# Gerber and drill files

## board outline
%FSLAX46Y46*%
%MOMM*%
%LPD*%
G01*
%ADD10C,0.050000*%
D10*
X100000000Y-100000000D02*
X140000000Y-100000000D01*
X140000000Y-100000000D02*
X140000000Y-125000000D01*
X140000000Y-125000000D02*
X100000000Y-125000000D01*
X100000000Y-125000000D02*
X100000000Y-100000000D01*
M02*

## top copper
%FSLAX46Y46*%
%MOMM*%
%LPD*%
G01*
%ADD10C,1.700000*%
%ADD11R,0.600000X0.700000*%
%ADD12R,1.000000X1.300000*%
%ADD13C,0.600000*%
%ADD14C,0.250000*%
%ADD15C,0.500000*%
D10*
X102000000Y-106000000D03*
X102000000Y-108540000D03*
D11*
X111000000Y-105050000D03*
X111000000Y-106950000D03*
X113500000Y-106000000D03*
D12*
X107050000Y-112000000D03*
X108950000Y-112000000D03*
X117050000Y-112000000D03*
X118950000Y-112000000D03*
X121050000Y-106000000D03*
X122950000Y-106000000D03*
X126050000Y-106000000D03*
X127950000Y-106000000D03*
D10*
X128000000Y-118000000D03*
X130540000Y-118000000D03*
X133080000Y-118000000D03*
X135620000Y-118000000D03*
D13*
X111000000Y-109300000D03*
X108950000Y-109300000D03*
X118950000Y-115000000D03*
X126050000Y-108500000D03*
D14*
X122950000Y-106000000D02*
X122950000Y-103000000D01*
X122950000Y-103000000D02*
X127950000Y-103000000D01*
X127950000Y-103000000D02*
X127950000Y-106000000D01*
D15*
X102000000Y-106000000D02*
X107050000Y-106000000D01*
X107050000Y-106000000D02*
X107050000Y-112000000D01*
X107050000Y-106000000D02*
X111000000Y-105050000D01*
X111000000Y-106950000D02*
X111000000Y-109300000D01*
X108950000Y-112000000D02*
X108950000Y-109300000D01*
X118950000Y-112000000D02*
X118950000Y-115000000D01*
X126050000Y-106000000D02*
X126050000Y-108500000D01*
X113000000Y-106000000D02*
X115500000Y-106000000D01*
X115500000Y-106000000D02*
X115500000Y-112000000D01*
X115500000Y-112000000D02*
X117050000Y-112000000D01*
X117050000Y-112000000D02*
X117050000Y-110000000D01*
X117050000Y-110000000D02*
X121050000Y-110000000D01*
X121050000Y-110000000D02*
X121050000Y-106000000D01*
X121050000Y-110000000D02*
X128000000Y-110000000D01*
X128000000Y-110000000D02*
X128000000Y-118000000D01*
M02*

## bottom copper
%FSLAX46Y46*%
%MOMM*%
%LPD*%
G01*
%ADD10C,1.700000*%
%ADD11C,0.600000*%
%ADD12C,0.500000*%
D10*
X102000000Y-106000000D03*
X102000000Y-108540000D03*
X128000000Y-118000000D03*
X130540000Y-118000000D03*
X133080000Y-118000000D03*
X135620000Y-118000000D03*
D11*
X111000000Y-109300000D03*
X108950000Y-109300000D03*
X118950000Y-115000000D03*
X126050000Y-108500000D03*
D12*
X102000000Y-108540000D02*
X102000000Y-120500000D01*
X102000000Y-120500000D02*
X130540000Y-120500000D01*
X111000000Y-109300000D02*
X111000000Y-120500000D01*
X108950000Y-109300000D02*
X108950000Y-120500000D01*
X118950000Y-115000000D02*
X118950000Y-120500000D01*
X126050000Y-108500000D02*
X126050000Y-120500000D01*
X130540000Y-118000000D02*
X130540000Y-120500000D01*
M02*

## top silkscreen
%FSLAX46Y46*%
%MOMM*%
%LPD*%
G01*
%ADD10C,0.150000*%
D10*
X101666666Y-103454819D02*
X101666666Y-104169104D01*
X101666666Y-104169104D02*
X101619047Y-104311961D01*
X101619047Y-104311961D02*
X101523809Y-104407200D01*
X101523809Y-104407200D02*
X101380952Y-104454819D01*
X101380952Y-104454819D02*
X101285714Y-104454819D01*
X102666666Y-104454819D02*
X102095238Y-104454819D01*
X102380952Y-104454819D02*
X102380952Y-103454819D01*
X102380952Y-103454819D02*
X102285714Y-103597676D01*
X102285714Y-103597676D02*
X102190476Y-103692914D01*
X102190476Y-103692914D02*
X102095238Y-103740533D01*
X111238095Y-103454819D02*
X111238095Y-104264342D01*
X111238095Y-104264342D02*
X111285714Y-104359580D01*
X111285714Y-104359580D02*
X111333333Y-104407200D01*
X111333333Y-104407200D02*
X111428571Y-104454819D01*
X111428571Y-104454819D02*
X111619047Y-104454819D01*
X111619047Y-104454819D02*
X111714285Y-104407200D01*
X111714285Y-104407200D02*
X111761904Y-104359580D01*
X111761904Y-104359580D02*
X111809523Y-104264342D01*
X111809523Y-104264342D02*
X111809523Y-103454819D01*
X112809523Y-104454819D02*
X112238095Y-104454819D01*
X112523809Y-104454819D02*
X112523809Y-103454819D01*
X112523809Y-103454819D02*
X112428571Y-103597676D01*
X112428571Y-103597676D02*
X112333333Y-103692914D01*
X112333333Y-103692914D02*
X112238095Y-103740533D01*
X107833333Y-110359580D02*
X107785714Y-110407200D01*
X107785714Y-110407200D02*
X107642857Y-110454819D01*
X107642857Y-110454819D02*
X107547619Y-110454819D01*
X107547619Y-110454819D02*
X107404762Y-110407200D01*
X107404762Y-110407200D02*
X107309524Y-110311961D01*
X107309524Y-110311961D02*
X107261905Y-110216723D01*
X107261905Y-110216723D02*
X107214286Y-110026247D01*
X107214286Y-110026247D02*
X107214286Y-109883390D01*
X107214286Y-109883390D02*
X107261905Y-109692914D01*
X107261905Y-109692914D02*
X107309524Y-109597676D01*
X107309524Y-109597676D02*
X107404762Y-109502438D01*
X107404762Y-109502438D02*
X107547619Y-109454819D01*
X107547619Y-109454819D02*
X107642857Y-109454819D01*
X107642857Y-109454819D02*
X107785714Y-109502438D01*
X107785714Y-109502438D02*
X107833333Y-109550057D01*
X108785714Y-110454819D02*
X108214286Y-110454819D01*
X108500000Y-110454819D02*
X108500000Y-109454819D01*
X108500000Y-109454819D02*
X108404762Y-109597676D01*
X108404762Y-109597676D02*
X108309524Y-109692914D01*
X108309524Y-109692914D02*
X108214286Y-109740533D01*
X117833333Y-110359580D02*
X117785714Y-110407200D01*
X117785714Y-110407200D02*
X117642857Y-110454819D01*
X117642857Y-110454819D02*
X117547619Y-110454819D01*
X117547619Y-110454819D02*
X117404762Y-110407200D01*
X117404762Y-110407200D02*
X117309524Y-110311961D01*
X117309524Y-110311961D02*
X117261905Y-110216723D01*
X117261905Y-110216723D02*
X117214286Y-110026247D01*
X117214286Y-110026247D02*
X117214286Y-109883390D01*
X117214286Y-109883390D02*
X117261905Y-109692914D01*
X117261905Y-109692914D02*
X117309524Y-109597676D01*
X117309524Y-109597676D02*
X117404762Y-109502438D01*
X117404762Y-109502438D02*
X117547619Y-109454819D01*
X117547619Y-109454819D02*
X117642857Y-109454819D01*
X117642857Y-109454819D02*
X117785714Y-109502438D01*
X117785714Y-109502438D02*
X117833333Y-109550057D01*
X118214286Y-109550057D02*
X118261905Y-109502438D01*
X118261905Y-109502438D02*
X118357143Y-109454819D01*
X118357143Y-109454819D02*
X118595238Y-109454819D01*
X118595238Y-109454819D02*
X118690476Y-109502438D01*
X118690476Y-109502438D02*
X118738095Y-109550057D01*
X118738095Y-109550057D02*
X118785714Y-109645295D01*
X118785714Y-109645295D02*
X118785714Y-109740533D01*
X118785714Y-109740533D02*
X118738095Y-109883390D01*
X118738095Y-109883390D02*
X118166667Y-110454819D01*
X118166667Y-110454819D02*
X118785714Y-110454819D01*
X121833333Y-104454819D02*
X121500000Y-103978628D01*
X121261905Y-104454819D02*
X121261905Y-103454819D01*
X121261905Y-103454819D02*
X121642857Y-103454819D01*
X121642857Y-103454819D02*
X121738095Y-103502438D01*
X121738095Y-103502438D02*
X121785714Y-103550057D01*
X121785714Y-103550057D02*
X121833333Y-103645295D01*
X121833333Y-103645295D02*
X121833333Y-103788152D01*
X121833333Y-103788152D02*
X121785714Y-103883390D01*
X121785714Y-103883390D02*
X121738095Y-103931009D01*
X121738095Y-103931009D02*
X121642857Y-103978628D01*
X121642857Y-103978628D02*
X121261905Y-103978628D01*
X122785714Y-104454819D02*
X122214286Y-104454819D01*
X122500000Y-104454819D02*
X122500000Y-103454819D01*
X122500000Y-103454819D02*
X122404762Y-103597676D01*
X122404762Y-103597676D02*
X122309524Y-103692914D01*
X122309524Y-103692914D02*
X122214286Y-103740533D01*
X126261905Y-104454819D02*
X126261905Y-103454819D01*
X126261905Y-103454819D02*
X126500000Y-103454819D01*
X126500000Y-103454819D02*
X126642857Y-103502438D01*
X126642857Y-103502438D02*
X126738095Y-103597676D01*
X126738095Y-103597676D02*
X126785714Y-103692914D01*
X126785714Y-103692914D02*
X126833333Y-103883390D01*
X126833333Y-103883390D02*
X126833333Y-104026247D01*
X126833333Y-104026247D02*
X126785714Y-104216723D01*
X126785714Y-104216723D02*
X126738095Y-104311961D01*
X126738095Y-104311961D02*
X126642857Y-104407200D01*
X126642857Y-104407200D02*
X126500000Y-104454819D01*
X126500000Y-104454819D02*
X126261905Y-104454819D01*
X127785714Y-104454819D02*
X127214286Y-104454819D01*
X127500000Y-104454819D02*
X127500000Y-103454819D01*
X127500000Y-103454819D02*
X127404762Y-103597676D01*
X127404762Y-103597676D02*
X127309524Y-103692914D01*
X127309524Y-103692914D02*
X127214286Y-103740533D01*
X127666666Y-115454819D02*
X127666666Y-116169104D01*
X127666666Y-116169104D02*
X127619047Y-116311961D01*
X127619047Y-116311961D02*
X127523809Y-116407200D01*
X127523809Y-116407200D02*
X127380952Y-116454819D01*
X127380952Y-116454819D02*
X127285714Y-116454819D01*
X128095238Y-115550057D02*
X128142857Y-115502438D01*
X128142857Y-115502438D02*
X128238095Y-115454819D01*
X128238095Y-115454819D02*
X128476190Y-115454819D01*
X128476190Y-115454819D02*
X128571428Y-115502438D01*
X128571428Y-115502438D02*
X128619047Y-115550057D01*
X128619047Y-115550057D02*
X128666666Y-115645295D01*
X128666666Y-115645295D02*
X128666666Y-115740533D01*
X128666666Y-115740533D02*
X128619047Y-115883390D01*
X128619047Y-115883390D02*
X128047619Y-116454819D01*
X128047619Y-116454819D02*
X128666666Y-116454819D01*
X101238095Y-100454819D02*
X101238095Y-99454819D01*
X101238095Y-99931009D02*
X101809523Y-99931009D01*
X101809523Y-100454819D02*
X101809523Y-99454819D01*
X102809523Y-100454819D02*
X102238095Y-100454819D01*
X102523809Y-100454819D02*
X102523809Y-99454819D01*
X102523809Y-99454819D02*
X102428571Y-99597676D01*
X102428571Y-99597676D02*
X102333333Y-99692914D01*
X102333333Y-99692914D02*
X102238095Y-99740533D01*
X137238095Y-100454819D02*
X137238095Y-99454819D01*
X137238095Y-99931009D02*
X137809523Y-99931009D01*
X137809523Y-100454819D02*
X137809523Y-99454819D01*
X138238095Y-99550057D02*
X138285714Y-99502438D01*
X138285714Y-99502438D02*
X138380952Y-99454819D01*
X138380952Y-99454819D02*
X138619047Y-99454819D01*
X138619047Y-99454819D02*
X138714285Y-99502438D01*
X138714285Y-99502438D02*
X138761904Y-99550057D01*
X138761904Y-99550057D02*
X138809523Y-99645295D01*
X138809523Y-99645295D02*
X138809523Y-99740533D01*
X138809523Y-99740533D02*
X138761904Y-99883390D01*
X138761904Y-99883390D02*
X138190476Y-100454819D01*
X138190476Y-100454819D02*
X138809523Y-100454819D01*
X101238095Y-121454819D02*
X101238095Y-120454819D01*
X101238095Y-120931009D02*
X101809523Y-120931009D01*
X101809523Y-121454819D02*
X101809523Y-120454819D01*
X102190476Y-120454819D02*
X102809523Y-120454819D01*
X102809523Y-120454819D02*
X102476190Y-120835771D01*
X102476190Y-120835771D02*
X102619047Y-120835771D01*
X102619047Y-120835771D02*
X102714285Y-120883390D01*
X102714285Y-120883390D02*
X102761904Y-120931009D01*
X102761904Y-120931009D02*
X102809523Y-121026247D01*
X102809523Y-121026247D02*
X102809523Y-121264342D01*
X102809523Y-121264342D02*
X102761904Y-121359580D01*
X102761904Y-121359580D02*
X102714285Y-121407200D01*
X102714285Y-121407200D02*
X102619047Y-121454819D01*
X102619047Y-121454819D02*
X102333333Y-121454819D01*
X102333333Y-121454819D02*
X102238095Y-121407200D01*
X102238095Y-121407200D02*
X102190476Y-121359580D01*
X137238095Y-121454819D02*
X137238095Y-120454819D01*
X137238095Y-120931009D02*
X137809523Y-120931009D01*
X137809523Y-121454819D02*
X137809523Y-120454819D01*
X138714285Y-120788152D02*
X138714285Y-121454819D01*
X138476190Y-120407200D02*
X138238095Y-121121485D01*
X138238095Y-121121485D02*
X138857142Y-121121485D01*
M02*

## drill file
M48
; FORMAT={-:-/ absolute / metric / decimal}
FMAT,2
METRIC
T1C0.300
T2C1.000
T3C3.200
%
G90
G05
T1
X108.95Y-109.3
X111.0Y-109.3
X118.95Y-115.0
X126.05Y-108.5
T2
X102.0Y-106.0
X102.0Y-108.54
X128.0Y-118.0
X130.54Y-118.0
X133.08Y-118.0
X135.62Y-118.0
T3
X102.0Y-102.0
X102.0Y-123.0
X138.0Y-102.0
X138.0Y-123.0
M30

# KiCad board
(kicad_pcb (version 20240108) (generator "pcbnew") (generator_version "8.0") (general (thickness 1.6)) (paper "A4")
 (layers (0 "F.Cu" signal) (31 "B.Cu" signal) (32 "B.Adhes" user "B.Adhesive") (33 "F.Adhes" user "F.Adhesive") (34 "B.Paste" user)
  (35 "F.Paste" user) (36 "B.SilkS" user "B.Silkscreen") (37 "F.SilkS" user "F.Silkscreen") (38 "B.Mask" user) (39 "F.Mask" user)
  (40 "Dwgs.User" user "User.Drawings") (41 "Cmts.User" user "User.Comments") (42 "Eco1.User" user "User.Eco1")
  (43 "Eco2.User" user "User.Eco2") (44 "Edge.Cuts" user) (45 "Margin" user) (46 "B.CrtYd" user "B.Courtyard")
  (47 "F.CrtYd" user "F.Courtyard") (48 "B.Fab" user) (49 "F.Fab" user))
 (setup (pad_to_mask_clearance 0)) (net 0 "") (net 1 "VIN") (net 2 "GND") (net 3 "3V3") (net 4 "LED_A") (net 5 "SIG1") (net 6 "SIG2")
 (gr_line (start 100 100) (end 140 100) (stroke (width 0.05) (type default)) (layer "Edge.Cuts"))
 (gr_line (start 140 100) (end 140 125) (stroke (width 0.05) (type default)) (layer "Edge.Cuts"))
 (gr_line (start 140 125) (end 100 125) (stroke (width 0.05) (type default)) (layer "Edge.Cuts"))
 (gr_line (start 100 125) (end 100 100) (stroke (width 0.05) (type default)) (layer "Edge.Cuts"))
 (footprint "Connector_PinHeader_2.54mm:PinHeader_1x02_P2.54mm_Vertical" (layer "F.Cu") (at 102 106)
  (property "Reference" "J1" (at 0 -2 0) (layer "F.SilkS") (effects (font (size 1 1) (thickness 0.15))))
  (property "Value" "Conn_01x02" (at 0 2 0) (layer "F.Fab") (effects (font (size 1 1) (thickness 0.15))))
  (pad "1" thru_hole circle (at 0 0) (size 1.7 1.7) (drill 1) (layers "*.Cu" "*.Mask") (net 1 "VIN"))
  (pad "2" thru_hole circle (at 0 2.54) (size 1.7 1.7) (drill 1) (layers "*.Cu" "*.Mask") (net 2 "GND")))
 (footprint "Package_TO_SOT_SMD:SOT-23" (layer "F.Cu") (at 112 106)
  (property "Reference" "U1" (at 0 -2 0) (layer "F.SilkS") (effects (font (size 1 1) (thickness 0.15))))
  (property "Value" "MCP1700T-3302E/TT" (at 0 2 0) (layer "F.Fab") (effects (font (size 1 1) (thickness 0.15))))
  (pad "1" smd rect (at -1 -0.95) (size 0.6 0.7) (layers "F.Cu" "F.Paste" "F.Mask") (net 1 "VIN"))
  (pad "2" smd rect (at -1 0.95) (size 0.6 0.7) (layers "F.Cu" "F.Paste" "F.Mask") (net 2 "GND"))
  (pad "3" smd rect (at 1.5 0) (size 0.6 0.7) (layers "F.Cu" "F.Paste" "F.Mask") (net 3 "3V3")))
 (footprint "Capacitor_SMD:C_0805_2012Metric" (layer "F.Cu") (at 108 112)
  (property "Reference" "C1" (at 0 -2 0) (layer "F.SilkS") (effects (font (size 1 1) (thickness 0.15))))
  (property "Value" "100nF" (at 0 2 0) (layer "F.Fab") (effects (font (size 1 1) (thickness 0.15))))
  (pad "1" smd rect (at -0.95 0) (size 1 1.3) (layers "F.Cu" "F.Paste" "F.Mask") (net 1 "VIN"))
  (pad "2" smd rect (at 0.95 0) (size 1 1.3) (layers "F.Cu" "F.Paste" "F.Mask") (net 2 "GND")))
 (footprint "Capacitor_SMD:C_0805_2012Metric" (layer "F.Cu") (at 118 112)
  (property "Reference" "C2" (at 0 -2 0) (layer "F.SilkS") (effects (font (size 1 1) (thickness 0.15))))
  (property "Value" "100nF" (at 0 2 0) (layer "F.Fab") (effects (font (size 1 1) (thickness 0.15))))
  (pad "1" smd rect (at -0.95 0) (size 1 1.3) (layers "F.Cu" "F.Paste" "F.Mask") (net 3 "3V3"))
  (pad "2" smd rect (at 0.95 0) (size 1 1.3) (layers "F.Cu" "F.Paste" "F.Mask") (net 2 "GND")))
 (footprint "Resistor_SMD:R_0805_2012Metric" (layer "F.Cu") (at 122 106)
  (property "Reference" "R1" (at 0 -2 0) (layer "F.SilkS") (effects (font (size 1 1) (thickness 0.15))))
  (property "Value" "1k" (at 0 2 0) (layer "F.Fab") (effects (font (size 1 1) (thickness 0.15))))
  (pad "1" smd rect (at -0.95 0) (size 1 1.3) (layers "F.Cu" "F.Paste" "F.Mask") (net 3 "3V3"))
  (pad "2" smd rect (at 0.95 0) (size 1 1.3) (layers "F.Cu" "F.Paste" "F.Mask") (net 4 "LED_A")))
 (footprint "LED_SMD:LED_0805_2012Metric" (layer "F.Cu") (at 127 106)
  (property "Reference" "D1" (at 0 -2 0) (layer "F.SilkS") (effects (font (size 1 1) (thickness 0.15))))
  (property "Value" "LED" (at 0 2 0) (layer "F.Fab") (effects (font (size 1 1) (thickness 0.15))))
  (pad "1" smd rect (at -0.95 0) (size 1 1.3) (layers "F.Cu" "F.Paste" "F.Mask") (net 2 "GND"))
  (pad "2" smd rect (at 0.95 0) (size 1 1.3) (layers "F.Cu" "F.Paste" "F.Mask") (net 4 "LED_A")))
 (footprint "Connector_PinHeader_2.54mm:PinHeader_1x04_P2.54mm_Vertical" (layer "F.Cu") (at 128 118)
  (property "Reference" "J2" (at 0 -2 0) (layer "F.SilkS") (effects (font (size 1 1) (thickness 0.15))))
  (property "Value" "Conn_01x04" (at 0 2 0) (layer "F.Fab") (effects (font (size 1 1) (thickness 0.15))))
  (pad "1" thru_hole circle (at 0 0) (size 1.7 1.7) (drill 1) (layers "*.Cu" "*.Mask") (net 3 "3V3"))
  (pad "2" thru_hole circle (at 2.54 0) (size 1.7 1.7) (drill 1) (layers "*.Cu" "*.Mask") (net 2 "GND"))
  (pad "3" thru_hole circle (at 5.08 0) (size 1.7 1.7) (drill 1) (layers "*.Cu" "*.Mask") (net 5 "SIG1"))
  (pad "4" thru_hole circle (at 7.62 0) (size 1.7 1.7) (drill 1) (layers "*.Cu" "*.Mask") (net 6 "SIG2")))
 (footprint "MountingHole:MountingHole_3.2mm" (layer "F.Cu") (at 102 102)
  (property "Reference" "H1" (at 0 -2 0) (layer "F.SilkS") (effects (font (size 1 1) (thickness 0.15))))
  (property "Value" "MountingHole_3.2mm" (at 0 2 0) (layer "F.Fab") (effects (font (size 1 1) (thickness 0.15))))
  (pad "1" np_thru_hole circle (at 0 0) (size 3.2 3.2) (drill 3.2) (layers "*.Cu" "*.Mask")))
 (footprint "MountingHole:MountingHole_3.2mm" (layer "F.Cu") (at 138 102)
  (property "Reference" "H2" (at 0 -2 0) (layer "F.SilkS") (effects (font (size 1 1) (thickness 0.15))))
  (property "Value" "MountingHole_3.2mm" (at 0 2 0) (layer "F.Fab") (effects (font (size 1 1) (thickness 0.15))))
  (pad "1" np_thru_hole circle (at 0 0) (size 3.2 3.2) (drill 3.2) (layers "*.Cu" "*.Mask")))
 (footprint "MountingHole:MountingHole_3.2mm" (layer "F.Cu") (at 102 123)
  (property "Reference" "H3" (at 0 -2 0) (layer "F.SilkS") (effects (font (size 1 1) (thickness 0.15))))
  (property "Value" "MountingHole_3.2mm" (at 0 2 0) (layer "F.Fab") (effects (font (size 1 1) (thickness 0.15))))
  (pad "1" np_thru_hole circle (at 0 0) (size 3.2 3.2) (drill 3.2) (layers "*.Cu" "*.Mask")))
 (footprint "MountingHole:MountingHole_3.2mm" (layer "F.Cu") (at 138 123)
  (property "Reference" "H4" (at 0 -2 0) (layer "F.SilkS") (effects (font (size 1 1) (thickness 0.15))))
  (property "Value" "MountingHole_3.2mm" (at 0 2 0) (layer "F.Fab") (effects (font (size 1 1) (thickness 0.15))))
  (pad "1" np_thru_hole circle (at 0 0) (size 3.2 3.2) (drill 3.2) (layers "*.Cu" "*.Mask")))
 (segment (start 122.95 106) (end 122.95 103) (width 0.25) (layer "F.Cu") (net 4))
 (segment (start 122.95 103) (end 127.95 103) (width 0.25) (layer "F.Cu") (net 4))
 (segment (start 127.95 103) (end 127.95 106) (width 0.25) (layer "F.Cu") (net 4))
 (segment (start 102 106) (end 107.05 106) (width 0.5) (layer "F.Cu") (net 1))
 (segment (start 107.05 106) (end 107.05 112) (width 0.5) (layer "F.Cu") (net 1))
 (segment (start 107.05 106) (end 111 105.05) (width 0.5) (layer "F.Cu") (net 1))
 (segment (start 111 106.95) (end 111 109.3) (width 0.5) (layer "F.Cu") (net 2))
 (segment (start 108.95 112) (end 108.95 109.3) (width 0.5) (layer "F.Cu") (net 2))
 (segment (start 118.95 112) (end 118.95 115) (width 0.5) (layer "F.Cu") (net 2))
 (segment (start 126.05 106) (end 126.05 108.5) (width 0.5) (layer "F.Cu") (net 2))
 (segment (start 113 106) (end 115.5 106) (width 0.5) (layer "F.Cu") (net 3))
 (segment (start 115.5 106) (end 115.5 112) (width 0.5) (layer "F.Cu") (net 3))
 (segment (start 115.5 112) (end 117.05 112) (width 0.5) (layer "F.Cu") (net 3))
 (segment (start 117.05 112) (end 117.05 110) (width 0.5) (layer "F.Cu") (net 3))
 (segment (start 117.05 110) (end 121.05 110) (width 0.5) (layer "F.Cu") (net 3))
 (segment (start 121.05 110) (end 121.05 106) (width 0.5) (layer "F.Cu") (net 3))
 (segment (start 121.05 110) (end 128 110) (width 0.5) (layer "F.Cu") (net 3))
 (segment (start 128 110) (end 128 118) (width 0.5) (layer "F.Cu") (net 3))
 (segment (start 102 108.54) (end 102 120.5) (width 0.5) (layer "B.Cu") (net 2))
 (segment (start 102 120.5) (end 130.54 120.5) (width 0.5) (layer "B.Cu") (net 2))
 (segment (start 111 109.3) (end 111 120.5) (width 0.5) (layer "B.Cu") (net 2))
 (segment (start 108.95 109.3) (end 108.95 120.5) (width 0.5) (layer "B.Cu") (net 2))
 (segment (start 118.95 115) (end 118.95 120.5) (width 0.5) (layer "B.Cu") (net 2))
 (segment (start 126.05 108.5) (end 126.05 120.5) (width 0.5) (layer "B.Cu") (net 2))
 (segment (start 130.54 118) (end 130.54 120.5) (width 0.5) (layer "B.Cu") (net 2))
 (via (at 111 109.3) (size 0.6) (drill 0.3) (layers "F.Cu" "B.Cu") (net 2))
 (via (at 108.95 109.3) (size 0.6) (drill 0.3) (layers "F.Cu" "B.Cu") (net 2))
 (via (at 118.95 115) (size 0.6) (drill 0.3) (layers "F.Cu" "B.Cu") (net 2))
 (via (at 126.05 108.5) (size 0.6) (drill 0.3) (layers "F.Cu" "B.Cu") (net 2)))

